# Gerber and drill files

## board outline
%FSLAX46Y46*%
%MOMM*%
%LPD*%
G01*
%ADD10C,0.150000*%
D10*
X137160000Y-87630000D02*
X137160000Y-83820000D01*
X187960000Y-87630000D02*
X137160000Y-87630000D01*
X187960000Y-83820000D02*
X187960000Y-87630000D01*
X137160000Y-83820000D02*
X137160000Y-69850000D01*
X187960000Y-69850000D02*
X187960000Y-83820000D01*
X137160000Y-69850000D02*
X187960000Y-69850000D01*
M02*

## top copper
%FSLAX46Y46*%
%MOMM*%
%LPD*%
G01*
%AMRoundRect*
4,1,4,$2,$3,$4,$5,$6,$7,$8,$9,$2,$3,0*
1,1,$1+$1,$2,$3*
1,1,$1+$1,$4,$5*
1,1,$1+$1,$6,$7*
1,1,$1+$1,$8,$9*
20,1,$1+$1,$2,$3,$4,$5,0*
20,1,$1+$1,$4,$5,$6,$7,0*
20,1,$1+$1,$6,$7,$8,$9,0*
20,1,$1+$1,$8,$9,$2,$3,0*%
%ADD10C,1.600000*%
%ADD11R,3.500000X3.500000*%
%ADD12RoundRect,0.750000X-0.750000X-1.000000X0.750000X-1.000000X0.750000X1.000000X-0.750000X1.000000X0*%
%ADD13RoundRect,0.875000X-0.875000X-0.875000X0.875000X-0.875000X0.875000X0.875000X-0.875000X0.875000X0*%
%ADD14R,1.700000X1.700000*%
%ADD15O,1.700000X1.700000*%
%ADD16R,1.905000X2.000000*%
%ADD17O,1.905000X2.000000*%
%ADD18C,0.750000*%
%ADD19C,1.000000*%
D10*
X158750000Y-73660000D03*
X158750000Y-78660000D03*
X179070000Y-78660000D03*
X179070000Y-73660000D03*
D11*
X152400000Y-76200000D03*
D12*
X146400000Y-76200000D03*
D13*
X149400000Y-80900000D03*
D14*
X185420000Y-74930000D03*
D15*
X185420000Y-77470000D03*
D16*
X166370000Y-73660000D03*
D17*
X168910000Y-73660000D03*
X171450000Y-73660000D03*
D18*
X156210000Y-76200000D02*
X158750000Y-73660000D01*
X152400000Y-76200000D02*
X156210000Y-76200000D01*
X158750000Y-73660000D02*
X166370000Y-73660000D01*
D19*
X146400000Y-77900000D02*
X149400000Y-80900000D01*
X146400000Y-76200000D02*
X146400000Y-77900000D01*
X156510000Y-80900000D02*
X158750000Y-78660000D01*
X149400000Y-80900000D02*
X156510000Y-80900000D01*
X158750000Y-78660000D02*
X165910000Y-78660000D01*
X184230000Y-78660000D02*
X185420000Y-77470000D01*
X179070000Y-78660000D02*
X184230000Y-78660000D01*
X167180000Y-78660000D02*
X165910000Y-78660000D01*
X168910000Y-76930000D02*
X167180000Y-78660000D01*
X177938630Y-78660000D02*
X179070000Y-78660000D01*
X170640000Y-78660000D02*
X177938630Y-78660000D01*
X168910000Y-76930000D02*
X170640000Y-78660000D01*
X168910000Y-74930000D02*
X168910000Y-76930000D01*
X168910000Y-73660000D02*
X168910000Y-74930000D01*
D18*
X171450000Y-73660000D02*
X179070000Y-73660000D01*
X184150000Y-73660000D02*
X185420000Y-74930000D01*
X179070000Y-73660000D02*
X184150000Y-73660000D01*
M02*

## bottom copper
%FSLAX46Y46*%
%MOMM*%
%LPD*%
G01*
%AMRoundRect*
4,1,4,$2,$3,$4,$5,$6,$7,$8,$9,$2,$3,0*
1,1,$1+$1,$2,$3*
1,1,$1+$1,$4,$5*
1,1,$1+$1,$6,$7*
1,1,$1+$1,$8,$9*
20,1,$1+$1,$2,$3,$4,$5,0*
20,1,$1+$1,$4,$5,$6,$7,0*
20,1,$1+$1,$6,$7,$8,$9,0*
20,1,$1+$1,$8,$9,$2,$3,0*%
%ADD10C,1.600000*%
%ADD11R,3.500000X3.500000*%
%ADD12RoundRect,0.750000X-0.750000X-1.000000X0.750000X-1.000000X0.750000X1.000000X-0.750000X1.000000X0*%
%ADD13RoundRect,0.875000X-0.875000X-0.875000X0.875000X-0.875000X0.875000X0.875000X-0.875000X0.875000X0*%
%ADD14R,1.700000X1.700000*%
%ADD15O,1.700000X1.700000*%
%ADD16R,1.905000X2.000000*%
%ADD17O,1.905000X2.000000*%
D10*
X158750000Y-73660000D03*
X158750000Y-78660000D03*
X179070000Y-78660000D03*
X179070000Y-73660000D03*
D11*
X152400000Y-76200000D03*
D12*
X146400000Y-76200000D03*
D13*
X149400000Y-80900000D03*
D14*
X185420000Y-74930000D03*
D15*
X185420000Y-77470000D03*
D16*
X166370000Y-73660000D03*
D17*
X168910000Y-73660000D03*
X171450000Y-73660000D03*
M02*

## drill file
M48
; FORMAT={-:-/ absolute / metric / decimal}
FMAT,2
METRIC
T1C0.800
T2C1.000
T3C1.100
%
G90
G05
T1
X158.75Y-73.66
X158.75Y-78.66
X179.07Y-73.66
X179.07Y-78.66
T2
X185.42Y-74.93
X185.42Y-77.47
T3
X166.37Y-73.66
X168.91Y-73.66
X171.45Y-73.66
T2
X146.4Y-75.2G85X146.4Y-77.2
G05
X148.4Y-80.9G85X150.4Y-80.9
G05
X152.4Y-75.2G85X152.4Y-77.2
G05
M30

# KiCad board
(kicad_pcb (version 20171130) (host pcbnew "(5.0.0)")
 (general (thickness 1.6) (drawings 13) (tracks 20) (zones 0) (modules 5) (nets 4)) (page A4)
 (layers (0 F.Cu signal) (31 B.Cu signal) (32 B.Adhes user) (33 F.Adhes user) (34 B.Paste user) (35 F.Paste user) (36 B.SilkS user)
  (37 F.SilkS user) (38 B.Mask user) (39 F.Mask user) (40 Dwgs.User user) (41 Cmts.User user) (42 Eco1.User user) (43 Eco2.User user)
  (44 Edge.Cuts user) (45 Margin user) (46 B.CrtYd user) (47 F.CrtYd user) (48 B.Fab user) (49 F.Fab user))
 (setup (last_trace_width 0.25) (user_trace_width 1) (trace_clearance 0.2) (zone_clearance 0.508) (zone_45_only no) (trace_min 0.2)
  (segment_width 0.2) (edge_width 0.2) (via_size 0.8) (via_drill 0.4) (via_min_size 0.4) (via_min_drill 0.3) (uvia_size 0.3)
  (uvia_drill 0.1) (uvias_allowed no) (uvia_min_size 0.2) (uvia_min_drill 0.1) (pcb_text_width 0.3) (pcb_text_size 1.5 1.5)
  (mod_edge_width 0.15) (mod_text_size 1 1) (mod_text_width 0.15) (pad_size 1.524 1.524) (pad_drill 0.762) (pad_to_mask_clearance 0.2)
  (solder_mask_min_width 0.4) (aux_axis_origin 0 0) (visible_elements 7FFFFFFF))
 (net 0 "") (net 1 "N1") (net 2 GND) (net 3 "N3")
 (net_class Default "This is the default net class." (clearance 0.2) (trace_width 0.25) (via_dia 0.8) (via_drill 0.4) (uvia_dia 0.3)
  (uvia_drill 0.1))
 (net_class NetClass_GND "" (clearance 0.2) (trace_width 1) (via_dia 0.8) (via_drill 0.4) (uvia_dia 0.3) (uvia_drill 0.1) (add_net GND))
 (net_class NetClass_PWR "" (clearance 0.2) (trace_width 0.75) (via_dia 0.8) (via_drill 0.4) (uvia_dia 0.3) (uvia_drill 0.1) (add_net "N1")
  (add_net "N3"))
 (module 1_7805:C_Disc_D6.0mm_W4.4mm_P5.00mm (layer F.Cu) (at 158.75 73.66 270)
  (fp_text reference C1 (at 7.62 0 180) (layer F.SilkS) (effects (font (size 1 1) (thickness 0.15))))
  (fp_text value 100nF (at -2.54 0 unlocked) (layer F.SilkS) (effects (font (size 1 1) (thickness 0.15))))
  (pad 1 thru_hole circle (at 0 0 270) (size 1.6 1.6) (drill 0.8) (layers *.Cu *.Mask) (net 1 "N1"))
  (pad 2 thru_hole circle (at 5 0 270) (size 1.6 1.6) (drill 0.8) (layers *.Cu *.Mask) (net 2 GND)))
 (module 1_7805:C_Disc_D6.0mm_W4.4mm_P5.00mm (layer F.Cu) (at 179.07 73.66 270)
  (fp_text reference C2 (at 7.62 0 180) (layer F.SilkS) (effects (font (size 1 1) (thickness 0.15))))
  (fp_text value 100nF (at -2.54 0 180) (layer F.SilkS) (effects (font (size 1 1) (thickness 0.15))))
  (pad 2 thru_hole circle (at 5 0 270) (size 1.6 1.6) (drill 0.8) (layers *.Cu *.Mask) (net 2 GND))
  (pad 1 thru_hole circle (at 0 0 270) (size 1.6 1.6) (drill 0.8) (layers *.Cu *.Mask) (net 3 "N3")))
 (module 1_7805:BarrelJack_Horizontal (layer F.Cu) (at 152.4 76.2)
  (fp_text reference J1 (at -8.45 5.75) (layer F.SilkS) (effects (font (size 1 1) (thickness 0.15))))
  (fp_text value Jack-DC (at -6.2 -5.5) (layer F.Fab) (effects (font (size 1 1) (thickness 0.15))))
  (pad 1 thru_hole rect (at 0 0) (size 3.5 3.5) (drill oval 1 3) (layers *.Cu *.Mask) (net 1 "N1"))
  (pad 2 thru_hole roundrect (at -6 0) (size 3 3.5) (drill oval 1 3) (layers *.Cu *.Mask) (roundrect_rratio 0.25) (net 2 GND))
  (pad 3 thru_hole roundrect (at -3 4.7) (size 3.5 3.5) (drill oval 3 1) (layers *.Cu *.Mask) (roundrect_rratio 0.25) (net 2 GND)))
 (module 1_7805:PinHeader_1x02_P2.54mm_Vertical (layer F.Cu) (at 185.42 74.93)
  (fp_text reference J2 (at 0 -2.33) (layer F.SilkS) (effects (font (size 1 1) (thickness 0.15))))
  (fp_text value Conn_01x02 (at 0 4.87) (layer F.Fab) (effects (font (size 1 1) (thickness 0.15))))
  (pad 1 thru_hole rect (at 0 0) (size 1.7 1.7) (drill 1) (layers *.Cu *.Mask) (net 3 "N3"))
  (pad 2 thru_hole oval (at 0 2.54) (size 1.7 1.7) (drill 1) (layers *.Cu *.Mask) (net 2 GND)))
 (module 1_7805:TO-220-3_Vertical (layer F.Cu) (at 166.37 73.66)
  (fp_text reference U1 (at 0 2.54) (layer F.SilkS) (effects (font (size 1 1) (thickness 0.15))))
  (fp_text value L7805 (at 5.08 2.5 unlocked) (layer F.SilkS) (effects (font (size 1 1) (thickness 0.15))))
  (pad 1 thru_hole rect (at 0 0) (size 1.905 2) (drill 1.1) (layers *.Cu *.Mask) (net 1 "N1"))
  (pad 2 thru_hole oval (at 2.54 0) (size 1.905 2) (drill 1.1) (layers *.Cu *.Mask) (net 2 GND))
  (pad 3 thru_hole oval (at 5.08 0) (size 1.905 2) (drill 1.1) (layers *.Cu *.Mask) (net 3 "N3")))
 (gr_line (start 137.16 87.63) (end 137.16 83.82) (layer Edge.Cuts) (width 0.15))
 (gr_line (start 187.96 87.63) (end 137.16 87.63) (layer Edge.Cuts) (width 0.15))
 (gr_line (start 187.96 83.82) (end 187.96 87.63) (layer Edge.Cuts) (width 0.15))
 (gr_line (start 137.16 83.82) (end 137.16 69.85) (layer Edge.Cuts) (width 0.15))
 (gr_line (start 187.96 69.85) (end 187.96 83.82) (layer Edge.Cuts) (width 0.15))
 (gr_line (start 137.16 69.85) (end 187.96 69.85) (layer Edge.Cuts) (width 0.15))
 (segment (start 156.21 76.2) (end 158.75 73.66) (width 0.75) (layer F.Cu) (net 1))
 (segment (start 152.4 76.2) (end 156.21 76.2) (width 0.75) (layer F.Cu) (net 1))
 (segment (start 158.75 73.66) (end 166.37 73.66) (width 0.75) (layer F.Cu) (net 1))
 (segment (start 146.4 77.9) (end 149.4 80.9) (width 1) (layer F.Cu) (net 2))
 (segment (start 146.4 76.2) (end 146.4 77.9) (width 1) (layer F.Cu) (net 2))
 (segment (start 156.51 80.9) (end 158.75 78.66) (width 1) (layer F.Cu) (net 2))
 (segment (start 149.4 80.9) (end 156.51 80.9) (width 1) (layer F.Cu) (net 2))
 (segment (start 158.75 78.66) (end 165.91 78.66) (width 1) (layer F.Cu) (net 2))
 (segment (start 184.23 78.66) (end 185.42 77.47) (width 1) (layer F.Cu) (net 2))
 (segment (start 179.07 78.66) (end 184.23 78.66) (width 1) (layer F.Cu) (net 2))
 (segment (start 167.18 78.66) (end 165.91 78.66) (width 1) (layer F.Cu) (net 2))
 (segment (start 168.91 76.93) (end 167.18 78.66) (width 1) (layer F.Cu) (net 2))
 (segment (start 177.93863 78.66) (end 179.07 78.66) (width 1) (layer F.Cu) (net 2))
 (segment (start 170.64 78.66) (end 177.93863 78.66) (width 1) (layer F.Cu) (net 2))
 (segment (start 168.91 76.93) (end 170.64 78.66) (width 1) (layer F.Cu) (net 2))
 (segment (start 168.91 74.93) (end 168.91 76.93) (width 1) (layer F.Cu) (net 2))
 (segment (start 168.91 73.66) (end 168.91 74.93) (width 1) (layer F.Cu) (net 2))
 (segment (start 171.45 73.66) (end 179.07 73.66) (width 0.75) (layer F.Cu) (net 3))
 (segment (start 184.15 73.66) (end 185.42 74.93) (width 0.75) (layer F.Cu) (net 3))
 (segment (start 179.07 73.66) (end 184.15 73.66) (width 0.75) (layer F.Cu) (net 3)))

